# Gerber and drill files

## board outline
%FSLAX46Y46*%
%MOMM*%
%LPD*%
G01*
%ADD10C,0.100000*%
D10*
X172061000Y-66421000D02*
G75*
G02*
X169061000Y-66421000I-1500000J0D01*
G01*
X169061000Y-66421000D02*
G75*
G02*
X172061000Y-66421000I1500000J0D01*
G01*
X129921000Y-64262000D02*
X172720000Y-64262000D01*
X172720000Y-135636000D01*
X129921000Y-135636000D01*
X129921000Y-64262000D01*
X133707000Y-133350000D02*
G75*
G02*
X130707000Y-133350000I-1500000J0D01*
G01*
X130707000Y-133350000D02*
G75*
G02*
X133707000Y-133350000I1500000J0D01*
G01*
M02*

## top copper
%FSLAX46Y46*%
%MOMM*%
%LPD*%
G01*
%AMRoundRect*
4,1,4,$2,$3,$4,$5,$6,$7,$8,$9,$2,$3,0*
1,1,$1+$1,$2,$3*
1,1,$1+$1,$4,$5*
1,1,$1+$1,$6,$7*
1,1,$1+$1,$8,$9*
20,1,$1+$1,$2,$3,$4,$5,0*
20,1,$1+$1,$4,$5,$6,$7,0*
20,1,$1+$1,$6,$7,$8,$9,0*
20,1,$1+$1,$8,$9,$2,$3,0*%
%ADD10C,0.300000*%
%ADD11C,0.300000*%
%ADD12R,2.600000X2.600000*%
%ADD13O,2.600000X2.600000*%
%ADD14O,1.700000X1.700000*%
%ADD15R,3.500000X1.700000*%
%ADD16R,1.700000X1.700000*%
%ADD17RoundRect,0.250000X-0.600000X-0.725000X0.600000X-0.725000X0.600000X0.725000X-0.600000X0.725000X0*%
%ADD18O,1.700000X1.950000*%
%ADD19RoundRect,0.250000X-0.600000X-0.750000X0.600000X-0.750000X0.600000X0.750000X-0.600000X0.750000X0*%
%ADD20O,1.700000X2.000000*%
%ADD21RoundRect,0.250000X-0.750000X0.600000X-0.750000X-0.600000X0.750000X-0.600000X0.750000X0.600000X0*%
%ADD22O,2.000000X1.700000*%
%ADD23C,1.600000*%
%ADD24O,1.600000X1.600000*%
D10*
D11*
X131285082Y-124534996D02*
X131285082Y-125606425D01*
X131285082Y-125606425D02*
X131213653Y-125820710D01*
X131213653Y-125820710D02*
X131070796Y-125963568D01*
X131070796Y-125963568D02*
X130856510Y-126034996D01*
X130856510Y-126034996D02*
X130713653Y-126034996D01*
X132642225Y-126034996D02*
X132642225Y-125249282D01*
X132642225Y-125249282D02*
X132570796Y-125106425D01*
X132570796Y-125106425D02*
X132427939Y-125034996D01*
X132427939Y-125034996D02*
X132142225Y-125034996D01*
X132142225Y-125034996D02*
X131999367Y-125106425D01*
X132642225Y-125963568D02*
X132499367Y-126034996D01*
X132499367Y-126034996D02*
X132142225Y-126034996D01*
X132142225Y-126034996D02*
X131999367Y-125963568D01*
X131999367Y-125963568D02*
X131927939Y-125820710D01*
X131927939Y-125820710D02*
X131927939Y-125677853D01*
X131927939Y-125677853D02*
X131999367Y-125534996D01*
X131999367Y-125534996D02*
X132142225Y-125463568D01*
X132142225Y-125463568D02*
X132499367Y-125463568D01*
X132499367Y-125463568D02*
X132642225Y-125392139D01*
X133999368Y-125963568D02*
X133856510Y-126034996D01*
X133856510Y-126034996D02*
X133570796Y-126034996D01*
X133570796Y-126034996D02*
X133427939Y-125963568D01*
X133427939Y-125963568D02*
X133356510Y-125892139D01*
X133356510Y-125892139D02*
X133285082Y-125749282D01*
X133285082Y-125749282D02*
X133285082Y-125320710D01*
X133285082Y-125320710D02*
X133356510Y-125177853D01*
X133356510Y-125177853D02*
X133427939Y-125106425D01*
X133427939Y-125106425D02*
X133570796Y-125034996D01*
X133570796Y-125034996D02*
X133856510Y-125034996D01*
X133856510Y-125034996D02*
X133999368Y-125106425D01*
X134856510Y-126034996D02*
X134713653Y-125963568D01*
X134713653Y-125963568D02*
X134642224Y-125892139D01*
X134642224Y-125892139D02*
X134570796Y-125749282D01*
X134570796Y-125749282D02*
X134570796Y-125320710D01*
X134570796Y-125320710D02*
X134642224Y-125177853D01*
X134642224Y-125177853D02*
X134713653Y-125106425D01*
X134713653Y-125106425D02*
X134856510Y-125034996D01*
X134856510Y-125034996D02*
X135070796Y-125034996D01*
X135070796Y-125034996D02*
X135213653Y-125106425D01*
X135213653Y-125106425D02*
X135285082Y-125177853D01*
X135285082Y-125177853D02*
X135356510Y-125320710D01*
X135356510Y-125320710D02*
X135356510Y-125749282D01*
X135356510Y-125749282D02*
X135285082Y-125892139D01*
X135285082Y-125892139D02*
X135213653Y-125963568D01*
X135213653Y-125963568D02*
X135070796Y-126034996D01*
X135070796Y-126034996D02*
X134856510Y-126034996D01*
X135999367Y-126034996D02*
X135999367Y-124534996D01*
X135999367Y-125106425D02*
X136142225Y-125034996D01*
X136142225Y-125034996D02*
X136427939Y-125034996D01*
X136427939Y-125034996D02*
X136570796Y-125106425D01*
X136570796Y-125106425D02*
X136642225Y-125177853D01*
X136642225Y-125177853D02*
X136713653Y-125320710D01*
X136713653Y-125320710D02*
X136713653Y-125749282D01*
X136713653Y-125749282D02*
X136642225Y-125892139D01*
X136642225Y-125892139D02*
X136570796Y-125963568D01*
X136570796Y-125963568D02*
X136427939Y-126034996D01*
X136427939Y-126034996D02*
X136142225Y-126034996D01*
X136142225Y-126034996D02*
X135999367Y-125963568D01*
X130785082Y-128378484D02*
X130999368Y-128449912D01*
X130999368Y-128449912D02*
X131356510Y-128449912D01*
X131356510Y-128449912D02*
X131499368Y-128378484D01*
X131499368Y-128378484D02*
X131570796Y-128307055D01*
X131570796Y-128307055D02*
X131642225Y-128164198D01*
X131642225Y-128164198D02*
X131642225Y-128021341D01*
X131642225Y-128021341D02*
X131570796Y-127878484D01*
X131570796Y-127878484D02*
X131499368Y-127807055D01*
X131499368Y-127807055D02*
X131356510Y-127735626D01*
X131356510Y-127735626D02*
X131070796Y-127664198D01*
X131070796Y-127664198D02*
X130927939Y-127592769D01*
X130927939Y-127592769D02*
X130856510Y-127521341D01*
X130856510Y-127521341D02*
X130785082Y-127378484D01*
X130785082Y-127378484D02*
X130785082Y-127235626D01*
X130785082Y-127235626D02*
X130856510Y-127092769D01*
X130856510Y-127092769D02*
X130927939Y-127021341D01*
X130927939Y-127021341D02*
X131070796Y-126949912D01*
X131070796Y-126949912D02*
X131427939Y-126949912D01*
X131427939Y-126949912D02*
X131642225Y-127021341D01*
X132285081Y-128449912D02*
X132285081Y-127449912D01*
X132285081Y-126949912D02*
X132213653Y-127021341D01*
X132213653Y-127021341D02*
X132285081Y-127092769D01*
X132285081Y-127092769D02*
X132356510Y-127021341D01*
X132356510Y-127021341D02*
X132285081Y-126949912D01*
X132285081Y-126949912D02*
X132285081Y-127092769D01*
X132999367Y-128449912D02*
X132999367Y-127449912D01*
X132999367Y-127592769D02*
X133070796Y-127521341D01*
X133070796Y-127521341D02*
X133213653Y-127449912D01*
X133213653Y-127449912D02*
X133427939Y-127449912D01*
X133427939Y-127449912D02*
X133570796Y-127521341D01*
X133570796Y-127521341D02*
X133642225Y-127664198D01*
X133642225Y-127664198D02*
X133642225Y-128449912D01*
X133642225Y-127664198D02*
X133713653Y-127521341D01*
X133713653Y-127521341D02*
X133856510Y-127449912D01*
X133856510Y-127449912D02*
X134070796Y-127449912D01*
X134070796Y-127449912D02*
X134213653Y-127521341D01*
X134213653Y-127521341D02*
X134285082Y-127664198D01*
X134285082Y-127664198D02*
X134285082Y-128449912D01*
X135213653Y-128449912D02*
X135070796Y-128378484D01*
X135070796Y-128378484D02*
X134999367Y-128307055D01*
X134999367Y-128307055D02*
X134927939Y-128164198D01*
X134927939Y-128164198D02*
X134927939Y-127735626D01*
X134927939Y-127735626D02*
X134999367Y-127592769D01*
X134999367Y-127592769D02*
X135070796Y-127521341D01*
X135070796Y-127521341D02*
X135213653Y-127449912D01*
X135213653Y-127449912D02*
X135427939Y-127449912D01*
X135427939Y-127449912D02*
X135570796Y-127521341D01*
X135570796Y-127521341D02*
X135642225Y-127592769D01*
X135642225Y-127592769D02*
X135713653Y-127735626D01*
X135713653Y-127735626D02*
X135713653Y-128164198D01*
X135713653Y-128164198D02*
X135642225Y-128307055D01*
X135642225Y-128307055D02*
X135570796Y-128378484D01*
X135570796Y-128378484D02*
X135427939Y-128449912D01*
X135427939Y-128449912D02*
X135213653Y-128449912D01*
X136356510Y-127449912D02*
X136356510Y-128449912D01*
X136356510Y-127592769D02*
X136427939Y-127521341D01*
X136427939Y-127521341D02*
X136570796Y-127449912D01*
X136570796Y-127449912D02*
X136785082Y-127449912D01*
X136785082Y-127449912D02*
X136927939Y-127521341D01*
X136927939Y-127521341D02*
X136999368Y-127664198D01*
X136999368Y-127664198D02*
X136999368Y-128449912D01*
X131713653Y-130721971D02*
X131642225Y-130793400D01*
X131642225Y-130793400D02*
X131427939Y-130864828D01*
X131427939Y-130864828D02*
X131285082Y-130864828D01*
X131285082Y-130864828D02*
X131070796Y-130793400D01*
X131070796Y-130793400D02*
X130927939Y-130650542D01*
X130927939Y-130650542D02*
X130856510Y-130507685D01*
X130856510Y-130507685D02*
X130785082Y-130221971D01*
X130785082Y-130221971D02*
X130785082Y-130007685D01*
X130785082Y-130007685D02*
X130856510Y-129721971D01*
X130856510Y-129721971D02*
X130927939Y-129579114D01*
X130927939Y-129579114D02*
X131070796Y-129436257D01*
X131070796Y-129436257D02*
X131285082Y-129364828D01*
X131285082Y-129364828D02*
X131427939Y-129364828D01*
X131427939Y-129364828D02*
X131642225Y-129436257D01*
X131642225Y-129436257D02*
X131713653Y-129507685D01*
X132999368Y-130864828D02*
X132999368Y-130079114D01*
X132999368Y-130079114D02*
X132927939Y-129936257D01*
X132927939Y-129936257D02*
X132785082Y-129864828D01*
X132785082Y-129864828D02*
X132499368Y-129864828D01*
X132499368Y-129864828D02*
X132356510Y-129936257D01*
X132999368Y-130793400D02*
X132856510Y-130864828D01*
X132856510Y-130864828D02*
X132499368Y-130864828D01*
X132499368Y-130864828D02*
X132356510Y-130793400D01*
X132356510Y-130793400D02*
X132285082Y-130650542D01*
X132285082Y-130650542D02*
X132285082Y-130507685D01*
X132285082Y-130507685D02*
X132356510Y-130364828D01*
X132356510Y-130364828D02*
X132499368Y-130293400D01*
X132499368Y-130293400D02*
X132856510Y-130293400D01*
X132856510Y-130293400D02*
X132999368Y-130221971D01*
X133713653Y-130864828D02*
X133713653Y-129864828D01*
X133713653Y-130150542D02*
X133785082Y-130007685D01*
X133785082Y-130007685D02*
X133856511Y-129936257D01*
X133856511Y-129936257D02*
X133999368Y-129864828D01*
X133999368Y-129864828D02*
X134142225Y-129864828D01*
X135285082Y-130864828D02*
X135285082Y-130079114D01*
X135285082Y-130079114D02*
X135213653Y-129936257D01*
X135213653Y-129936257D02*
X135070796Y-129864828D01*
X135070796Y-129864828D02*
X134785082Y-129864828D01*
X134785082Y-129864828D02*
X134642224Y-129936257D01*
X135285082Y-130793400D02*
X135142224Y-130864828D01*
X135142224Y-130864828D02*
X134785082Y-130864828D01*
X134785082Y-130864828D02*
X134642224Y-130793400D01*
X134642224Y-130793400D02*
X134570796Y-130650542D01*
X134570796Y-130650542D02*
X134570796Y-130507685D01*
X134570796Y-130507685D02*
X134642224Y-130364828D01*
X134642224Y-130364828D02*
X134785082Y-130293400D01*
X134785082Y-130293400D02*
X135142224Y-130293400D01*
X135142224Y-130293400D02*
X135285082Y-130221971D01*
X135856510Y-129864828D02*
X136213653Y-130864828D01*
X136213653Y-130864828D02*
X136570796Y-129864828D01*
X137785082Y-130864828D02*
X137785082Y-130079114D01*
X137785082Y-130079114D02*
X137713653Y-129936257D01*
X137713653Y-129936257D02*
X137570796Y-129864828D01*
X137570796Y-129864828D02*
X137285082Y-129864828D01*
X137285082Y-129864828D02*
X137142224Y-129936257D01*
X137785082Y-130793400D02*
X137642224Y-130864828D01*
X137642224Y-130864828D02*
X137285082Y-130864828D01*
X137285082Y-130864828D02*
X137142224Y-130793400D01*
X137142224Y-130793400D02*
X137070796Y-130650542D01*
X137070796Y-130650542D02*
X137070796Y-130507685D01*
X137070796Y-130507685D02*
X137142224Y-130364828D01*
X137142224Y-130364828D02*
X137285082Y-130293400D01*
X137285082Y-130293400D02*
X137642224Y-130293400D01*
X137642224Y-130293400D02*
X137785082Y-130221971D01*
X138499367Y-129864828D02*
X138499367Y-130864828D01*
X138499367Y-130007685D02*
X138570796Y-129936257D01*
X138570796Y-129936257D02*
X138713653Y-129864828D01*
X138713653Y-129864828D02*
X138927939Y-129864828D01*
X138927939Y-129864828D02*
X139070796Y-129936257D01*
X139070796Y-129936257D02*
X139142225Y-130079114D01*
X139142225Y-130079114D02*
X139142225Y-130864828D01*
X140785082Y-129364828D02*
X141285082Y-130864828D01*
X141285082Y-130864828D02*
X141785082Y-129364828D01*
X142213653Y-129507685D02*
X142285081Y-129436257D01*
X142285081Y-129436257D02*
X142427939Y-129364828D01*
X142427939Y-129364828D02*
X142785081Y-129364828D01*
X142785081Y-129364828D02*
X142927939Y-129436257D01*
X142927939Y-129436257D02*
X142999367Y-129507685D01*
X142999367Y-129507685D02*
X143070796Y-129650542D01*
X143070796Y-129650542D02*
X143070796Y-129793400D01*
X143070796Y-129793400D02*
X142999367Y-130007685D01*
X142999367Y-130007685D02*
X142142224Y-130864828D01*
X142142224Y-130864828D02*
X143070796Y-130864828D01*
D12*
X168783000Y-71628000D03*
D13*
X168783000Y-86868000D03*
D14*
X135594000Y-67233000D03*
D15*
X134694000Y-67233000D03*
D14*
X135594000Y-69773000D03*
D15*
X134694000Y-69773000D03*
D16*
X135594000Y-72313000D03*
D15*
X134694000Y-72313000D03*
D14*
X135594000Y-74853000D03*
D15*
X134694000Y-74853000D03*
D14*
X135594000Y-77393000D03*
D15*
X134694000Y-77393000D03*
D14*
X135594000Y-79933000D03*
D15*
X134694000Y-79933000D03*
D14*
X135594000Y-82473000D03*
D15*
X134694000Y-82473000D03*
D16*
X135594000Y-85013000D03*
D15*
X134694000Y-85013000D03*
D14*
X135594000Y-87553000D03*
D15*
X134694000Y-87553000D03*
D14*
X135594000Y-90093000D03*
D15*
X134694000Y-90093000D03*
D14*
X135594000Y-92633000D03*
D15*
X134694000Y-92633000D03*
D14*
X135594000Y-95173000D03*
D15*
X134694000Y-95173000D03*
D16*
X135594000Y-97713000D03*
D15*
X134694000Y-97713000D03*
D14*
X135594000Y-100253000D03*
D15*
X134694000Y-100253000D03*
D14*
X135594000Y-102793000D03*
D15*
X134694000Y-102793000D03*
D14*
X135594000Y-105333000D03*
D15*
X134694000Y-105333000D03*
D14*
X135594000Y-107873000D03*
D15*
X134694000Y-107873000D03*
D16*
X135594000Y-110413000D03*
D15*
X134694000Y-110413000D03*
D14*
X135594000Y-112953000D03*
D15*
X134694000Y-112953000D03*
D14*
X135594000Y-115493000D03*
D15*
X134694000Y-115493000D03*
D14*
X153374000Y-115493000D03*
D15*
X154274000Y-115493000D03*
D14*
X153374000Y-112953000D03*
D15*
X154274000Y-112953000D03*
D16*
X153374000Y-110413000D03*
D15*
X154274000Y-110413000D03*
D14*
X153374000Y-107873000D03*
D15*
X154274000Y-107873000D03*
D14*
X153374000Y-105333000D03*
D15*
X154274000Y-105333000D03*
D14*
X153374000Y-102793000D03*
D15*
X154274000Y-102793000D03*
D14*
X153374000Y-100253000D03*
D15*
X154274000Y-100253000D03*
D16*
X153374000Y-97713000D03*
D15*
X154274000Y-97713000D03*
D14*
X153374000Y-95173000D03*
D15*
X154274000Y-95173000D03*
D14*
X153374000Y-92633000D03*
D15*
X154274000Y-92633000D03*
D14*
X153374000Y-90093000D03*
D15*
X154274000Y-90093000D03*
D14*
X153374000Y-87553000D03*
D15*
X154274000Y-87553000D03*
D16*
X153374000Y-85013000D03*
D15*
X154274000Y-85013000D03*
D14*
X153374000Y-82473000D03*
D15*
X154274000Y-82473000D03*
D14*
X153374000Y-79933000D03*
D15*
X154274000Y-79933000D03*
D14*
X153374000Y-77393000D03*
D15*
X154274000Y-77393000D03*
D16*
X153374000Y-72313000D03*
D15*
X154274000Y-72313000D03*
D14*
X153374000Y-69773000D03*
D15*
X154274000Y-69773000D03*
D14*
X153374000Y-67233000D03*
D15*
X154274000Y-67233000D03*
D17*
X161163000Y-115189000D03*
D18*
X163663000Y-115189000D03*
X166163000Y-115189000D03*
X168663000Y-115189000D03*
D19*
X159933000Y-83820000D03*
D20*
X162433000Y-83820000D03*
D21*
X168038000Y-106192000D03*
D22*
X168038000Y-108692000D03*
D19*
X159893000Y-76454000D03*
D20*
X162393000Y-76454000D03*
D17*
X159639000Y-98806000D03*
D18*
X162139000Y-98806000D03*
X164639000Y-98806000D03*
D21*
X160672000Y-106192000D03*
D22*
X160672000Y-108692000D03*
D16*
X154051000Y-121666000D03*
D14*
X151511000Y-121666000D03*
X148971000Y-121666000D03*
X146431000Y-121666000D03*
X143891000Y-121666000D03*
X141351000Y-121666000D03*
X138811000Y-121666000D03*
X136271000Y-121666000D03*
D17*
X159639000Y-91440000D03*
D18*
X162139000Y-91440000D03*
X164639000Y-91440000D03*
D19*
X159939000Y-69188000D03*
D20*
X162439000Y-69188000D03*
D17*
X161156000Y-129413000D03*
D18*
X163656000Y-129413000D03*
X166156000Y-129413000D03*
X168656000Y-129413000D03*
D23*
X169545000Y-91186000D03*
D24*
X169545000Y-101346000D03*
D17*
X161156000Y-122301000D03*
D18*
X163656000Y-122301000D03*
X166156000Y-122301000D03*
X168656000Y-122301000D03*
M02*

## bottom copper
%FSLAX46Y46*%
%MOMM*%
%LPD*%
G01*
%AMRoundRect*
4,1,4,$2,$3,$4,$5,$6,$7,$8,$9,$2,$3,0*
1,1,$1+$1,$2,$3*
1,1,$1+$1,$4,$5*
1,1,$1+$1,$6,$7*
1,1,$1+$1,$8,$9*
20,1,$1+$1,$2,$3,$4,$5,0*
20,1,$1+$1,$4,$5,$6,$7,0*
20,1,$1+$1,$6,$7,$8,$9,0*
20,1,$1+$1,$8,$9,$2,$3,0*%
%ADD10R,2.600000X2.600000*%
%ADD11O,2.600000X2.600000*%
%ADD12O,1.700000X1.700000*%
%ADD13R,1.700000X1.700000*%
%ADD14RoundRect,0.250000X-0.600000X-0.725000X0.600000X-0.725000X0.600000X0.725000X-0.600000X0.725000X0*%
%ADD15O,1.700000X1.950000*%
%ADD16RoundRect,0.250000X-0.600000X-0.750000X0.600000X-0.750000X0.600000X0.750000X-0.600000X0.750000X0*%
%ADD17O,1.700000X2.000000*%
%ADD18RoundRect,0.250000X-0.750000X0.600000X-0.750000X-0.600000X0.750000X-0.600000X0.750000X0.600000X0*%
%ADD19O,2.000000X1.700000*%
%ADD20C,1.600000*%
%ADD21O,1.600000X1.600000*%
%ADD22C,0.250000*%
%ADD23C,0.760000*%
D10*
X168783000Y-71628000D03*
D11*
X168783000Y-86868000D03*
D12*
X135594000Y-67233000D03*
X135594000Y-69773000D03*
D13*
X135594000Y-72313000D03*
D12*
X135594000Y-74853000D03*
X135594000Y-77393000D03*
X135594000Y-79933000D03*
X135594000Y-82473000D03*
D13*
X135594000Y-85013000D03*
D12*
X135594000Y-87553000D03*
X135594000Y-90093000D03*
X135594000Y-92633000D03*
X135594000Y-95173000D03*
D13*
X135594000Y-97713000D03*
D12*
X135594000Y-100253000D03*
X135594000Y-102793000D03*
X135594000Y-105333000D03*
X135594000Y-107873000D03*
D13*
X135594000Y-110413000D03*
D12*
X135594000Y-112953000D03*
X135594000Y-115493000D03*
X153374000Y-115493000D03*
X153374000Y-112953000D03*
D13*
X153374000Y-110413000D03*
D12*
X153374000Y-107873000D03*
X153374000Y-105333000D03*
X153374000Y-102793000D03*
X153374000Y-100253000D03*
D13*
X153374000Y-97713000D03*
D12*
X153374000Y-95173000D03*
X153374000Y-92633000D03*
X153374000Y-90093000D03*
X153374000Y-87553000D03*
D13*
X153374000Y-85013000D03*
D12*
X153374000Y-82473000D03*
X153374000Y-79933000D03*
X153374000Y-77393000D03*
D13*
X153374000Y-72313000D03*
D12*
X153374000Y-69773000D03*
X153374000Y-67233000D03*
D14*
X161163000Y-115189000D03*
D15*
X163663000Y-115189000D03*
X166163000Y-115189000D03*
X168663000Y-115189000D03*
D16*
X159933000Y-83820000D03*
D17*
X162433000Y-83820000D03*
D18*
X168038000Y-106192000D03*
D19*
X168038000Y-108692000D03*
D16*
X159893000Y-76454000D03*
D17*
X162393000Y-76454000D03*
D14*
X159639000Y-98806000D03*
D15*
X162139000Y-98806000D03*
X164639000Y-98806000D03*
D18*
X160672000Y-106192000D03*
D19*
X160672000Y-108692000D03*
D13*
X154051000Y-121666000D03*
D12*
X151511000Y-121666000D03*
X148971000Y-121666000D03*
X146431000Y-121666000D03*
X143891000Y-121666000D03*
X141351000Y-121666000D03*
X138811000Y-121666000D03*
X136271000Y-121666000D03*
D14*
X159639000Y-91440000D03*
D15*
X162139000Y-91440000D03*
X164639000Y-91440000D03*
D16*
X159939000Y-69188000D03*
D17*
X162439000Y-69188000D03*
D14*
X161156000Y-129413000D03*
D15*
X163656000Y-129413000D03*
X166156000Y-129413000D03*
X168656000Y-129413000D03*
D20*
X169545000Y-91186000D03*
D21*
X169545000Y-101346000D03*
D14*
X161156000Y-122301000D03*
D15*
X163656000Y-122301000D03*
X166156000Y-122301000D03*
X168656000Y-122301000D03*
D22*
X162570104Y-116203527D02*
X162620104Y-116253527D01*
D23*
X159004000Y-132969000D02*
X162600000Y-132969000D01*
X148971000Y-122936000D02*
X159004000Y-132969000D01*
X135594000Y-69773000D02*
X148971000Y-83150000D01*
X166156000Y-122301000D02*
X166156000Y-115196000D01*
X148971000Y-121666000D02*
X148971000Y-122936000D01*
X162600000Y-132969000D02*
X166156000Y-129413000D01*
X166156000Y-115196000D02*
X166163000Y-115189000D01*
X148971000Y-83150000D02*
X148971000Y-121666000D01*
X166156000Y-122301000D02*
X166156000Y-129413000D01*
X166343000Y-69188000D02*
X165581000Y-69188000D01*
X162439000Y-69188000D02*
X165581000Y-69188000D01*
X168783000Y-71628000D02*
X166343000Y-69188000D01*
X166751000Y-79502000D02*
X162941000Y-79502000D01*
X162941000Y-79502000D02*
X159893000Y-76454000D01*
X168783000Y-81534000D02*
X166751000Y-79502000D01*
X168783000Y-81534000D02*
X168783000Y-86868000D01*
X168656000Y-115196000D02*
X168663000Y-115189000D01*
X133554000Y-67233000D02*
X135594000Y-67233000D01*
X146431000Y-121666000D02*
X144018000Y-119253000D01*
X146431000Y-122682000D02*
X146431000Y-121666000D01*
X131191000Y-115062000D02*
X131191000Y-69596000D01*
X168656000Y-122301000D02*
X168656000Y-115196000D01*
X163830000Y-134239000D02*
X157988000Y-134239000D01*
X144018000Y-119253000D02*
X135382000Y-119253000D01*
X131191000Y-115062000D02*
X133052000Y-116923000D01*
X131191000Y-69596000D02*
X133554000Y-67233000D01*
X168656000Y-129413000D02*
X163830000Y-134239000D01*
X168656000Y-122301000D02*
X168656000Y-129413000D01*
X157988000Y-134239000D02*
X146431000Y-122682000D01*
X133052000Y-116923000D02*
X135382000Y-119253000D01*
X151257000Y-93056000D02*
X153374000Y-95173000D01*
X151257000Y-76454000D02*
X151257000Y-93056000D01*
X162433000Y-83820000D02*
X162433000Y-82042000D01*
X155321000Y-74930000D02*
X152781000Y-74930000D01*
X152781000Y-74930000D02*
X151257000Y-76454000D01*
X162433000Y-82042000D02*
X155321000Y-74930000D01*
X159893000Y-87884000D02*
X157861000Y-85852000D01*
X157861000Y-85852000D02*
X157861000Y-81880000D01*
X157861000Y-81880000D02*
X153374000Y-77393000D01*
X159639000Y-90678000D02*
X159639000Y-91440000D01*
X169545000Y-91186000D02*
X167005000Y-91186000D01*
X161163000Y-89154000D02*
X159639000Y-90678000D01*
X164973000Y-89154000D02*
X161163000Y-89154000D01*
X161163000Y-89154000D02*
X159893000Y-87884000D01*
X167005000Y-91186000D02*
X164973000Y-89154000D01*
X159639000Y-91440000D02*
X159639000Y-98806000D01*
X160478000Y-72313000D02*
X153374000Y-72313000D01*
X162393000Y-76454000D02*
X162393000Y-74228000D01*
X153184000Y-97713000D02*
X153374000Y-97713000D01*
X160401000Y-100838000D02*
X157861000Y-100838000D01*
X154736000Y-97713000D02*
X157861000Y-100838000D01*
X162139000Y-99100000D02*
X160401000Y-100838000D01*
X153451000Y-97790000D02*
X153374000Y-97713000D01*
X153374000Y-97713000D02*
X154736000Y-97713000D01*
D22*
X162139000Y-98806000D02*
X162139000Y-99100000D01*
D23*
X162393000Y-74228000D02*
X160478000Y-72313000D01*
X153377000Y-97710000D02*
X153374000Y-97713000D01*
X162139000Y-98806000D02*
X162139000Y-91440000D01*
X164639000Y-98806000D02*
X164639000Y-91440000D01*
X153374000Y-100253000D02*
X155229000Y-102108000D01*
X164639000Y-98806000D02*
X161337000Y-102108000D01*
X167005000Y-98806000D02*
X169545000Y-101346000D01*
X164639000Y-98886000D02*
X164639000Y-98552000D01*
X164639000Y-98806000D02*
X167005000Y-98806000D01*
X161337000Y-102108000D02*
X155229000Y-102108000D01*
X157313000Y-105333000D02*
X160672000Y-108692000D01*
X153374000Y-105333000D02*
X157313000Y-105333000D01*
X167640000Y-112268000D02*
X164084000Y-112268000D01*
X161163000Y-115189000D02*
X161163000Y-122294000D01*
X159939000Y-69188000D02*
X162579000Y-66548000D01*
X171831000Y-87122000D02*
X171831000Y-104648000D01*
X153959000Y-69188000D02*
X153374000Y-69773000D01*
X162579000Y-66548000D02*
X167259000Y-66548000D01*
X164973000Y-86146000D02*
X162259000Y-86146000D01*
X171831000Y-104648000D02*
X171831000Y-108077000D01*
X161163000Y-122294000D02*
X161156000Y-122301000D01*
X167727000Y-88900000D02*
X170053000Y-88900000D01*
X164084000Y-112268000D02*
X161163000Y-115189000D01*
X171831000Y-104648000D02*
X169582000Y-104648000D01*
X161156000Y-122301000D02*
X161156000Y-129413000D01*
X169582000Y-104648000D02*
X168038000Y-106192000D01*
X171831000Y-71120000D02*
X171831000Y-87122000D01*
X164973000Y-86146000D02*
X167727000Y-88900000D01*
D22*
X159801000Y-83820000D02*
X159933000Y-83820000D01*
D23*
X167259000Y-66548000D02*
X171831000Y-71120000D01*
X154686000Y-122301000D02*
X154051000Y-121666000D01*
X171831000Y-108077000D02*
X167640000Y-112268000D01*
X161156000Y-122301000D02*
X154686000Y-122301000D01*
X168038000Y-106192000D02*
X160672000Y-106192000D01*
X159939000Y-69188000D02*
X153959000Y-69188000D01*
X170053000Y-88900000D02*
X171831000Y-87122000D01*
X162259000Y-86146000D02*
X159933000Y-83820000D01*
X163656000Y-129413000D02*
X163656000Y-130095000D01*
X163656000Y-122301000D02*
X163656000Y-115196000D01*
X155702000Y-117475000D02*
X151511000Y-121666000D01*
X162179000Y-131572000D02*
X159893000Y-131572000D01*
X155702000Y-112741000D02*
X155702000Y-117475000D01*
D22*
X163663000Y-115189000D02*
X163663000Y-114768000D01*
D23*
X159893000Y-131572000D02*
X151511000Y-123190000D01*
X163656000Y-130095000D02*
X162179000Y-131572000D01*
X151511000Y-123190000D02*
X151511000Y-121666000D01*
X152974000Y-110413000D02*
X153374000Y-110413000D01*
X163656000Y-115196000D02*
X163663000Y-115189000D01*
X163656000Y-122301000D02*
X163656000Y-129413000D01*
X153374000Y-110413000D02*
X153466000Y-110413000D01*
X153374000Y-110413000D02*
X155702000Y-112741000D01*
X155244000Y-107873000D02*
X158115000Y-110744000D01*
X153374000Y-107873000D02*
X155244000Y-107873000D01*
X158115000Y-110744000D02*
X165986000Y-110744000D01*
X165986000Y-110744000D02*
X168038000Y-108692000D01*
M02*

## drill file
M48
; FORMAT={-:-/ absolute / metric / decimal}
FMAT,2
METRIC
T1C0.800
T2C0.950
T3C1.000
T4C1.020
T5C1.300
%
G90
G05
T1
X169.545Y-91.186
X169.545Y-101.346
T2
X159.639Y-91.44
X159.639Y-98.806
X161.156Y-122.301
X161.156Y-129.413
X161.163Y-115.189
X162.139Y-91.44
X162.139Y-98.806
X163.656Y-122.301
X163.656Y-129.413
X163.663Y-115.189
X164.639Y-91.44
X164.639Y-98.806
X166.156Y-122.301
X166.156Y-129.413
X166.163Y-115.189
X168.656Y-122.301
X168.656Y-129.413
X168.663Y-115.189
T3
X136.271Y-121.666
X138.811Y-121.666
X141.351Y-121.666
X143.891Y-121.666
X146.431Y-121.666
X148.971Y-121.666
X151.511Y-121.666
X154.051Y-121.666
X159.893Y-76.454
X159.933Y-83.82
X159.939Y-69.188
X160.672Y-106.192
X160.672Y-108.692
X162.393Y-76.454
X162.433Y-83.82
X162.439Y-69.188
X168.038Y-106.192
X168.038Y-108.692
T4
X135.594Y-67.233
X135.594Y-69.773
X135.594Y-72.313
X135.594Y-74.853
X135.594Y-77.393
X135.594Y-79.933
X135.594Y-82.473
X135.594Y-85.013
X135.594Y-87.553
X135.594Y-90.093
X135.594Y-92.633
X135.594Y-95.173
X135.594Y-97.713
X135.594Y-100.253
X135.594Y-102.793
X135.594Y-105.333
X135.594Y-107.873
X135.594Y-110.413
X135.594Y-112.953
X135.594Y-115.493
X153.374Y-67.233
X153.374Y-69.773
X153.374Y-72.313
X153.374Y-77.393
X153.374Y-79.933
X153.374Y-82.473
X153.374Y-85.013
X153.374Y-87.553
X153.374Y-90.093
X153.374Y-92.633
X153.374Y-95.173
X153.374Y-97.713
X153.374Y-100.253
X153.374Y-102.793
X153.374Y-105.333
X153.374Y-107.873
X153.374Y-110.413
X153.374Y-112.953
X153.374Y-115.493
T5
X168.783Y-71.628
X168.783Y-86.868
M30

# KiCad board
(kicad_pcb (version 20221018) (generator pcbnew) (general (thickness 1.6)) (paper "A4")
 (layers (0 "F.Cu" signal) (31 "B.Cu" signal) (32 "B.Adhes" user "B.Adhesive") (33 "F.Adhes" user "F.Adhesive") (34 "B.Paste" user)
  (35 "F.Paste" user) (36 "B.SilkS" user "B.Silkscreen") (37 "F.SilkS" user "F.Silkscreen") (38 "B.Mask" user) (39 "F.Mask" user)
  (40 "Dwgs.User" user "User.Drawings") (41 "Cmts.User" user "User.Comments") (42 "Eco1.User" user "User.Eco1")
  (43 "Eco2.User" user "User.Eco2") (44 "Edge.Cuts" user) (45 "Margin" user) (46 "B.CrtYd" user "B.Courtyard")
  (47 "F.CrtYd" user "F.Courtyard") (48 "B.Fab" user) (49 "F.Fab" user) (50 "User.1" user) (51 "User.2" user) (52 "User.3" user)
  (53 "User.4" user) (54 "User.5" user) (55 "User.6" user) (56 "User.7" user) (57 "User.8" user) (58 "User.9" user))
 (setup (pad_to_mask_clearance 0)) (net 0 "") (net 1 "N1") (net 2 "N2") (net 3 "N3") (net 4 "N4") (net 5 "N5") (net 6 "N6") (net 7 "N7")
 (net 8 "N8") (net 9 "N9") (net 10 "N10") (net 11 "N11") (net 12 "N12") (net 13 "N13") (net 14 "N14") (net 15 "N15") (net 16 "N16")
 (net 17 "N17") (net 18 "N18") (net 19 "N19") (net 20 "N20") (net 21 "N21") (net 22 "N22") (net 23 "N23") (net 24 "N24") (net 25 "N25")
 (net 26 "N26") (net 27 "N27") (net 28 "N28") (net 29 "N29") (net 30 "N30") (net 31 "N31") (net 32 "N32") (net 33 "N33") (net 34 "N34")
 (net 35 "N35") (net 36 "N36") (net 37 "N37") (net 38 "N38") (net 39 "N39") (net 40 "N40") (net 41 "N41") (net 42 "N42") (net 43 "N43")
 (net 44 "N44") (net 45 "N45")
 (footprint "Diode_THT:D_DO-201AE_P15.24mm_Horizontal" (layer "F.Cu") (at 168.783 71.628 -90)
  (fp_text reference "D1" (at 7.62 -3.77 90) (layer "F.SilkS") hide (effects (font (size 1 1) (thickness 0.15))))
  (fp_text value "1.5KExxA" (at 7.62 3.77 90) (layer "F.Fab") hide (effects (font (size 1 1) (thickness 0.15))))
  (pad "1" thru_hole rect (at 0 0 270) (size 2.6 2.6) (drill 1.3) (layers "*.Cu" "*.Mask") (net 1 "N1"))
  (pad "2" thru_hole oval (at 15.24 0 270) (size 2.6 2.6) (drill 1.3) (layers "*.Cu" "*.Mask") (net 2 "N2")))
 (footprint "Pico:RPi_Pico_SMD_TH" (layer "F.Cu") (at 144.484 91.363)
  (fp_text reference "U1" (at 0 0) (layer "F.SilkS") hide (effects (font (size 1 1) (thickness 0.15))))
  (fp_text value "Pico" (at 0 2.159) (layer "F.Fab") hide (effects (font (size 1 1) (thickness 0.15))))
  (pad "1" thru_hole oval (at -8.89 -24.13) (size 1.7 1.7) (drill 1.02) (layers "*.Cu" "*.Mask") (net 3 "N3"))
  (pad "1" smd rect (at -8.89 -24.13) (size 3.5 1.7) (drill (offset -0.9 0)) (layers "F.Cu" "F.Mask") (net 3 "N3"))
  (pad "2" thru_hole oval (at -8.89 -21.59) (size 1.7 1.7) (drill 1.02) (layers "*.Cu" "*.Mask") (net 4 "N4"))
  (pad "2" smd rect (at -8.89 -21.59) (size 3.5 1.7) (drill (offset -0.9 0)) (layers "F.Cu" "F.Mask") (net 4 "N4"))
  (pad "3" thru_hole rect (at -8.89 -19.05) (size 1.7 1.7) (drill 1.02) (layers "*.Cu" "*.Mask") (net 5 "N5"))
  (pad "3" smd rect (at -8.89 -19.05) (size 3.5 1.7) (drill (offset -0.9 0)) (layers "F.Cu" "F.Mask") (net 5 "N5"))
  (pad "4" thru_hole oval (at -8.89 -16.51) (size 1.7 1.7) (drill 1.02) (layers "*.Cu" "*.Mask") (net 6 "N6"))
  (pad "4" smd rect (at -8.89 -16.51) (size 3.5 1.7) (drill (offset -0.9 0)) (layers "F.Cu" "F.Mask") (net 6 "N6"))
  (pad "5" thru_hole oval (at -8.89 -13.97) (size 1.7 1.7) (drill 1.02) (layers "*.Cu" "*.Mask") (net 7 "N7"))
  (pad "5" smd rect (at -8.89 -13.97) (size 3.5 1.7) (drill (offset -0.9 0)) (layers "F.Cu" "F.Mask") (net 7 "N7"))
  (pad "6" thru_hole oval (at -8.89 -11.43) (size 1.7 1.7) (drill 1.02) (layers "*.Cu" "*.Mask") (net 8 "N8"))
  (pad "6" smd rect (at -8.89 -11.43) (size 3.5 1.7) (drill (offset -0.9 0)) (layers "F.Cu" "F.Mask") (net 8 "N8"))
  (pad "7" thru_hole oval (at -8.89 -8.89) (size 1.7 1.7) (drill 1.02) (layers "*.Cu" "*.Mask") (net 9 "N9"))
  (pad "7" smd rect (at -8.89 -8.89) (size 3.5 1.7) (drill (offset -0.9 0)) (layers "F.Cu" "F.Mask") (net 9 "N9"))
  (pad "8" thru_hole rect (at -8.89 -6.35) (size 1.7 1.7) (drill 1.02) (layers "*.Cu" "*.Mask") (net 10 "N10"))
  (pad "8" smd rect (at -8.89 -6.35) (size 3.5 1.7) (drill (offset -0.9 0)) (layers "F.Cu" "F.Mask") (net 10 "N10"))
  (pad "9" thru_hole oval (at -8.89 -3.81) (size 1.7 1.7) (drill 1.02) (layers "*.Cu" "*.Mask") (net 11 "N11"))
  (pad "9" smd rect (at -8.89 -3.81) (size 3.5 1.7) (drill (offset -0.9 0)) (layers "F.Cu" "F.Mask") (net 11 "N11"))
  (pad "10" thru_hole oval (at -8.89 -1.27) (size 1.7 1.7) (drill 1.02) (layers "*.Cu" "*.Mask") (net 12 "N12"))
  (pad "10" smd rect (at -8.89 -1.27) (size 3.5 1.7) (drill (offset -0.9 0)) (layers "F.Cu" "F.Mask") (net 12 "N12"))
  (pad "11" thru_hole oval (at -8.89 1.27) (size 1.7 1.7) (drill 1.02) (layers "*.Cu" "*.Mask") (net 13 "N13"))
  (pad "11" smd rect (at -8.89 1.27) (size 3.5 1.7) (drill (offset -0.9 0)) (layers "F.Cu" "F.Mask") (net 13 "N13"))
  (pad "12" thru_hole oval (at -8.89 3.81) (size 1.7 1.7) (drill 1.02) (layers "*.Cu" "*.Mask") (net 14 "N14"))
  (pad "12" smd rect (at -8.89 3.81) (size 3.5 1.7) (drill (offset -0.9 0)) (layers "F.Cu" "F.Mask") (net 14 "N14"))
  (pad "13" thru_hole rect (at -8.89 6.35) (size 1.7 1.7) (drill 1.02) (layers "*.Cu" "*.Mask") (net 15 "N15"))
  (pad "13" smd rect (at -8.89 6.35) (size 3.5 1.7) (drill (offset -0.9 0)) (layers "F.Cu" "F.Mask") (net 15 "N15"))
  (pad "14" thru_hole oval (at -8.89 8.89) (size 1.7 1.7) (drill 1.02) (layers "*.Cu" "*.Mask") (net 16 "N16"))
  (pad "14" smd rect (at -8.89 8.89) (size 3.5 1.7) (drill (offset -0.9 0)) (layers "F.Cu" "F.Mask") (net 16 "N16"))
  (pad "15" thru_hole oval (at -8.89 11.43) (size 1.7 1.7) (drill 1.02) (layers "*.Cu" "*.Mask") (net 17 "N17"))
  (pad "15" smd rect (at -8.89 11.43) (size 3.5 1.7) (drill (offset -0.9 0)) (layers "F.Cu" "F.Mask") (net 17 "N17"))
  (pad "16" thru_hole oval (at -8.89 13.97) (size 1.7 1.7) (drill 1.02) (layers "*.Cu" "*.Mask") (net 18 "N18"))
  (pad "16" smd rect (at -8.89 13.97) (size 3.5 1.7) (drill (offset -0.9 0)) (layers "F.Cu" "F.Mask") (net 18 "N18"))
  (pad "17" thru_hole oval (at -8.89 16.51) (size 1.7 1.7) (drill 1.02) (layers "*.Cu" "*.Mask") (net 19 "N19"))
  (pad "17" smd rect (at -8.89 16.51) (size 3.5 1.7) (drill (offset -0.9 0)) (layers "F.Cu" "F.Mask") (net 19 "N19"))
  (pad "18" thru_hole rect (at -8.89 19.05) (size 1.7 1.7) (drill 1.02) (layers "*.Cu" "*.Mask") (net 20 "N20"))
  (pad "18" smd rect (at -8.89 19.05) (size 3.5 1.7) (drill (offset -0.9 0)) (layers "F.Cu" "F.Mask") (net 20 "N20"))
  (pad "19" thru_hole oval (at -8.89 21.59) (size 1.7 1.7) (drill 1.02) (layers "*.Cu" "*.Mask") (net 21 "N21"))
  (pad "19" smd rect (at -8.89 21.59) (size 3.5 1.7) (drill (offset -0.9 0)) (layers "F.Cu" "F.Mask") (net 21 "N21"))
  (pad "20" thru_hole oval (at -8.89 24.13) (size 1.7 1.7) (drill 1.02) (layers "*.Cu" "*.Mask") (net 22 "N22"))
  (pad "20" smd rect (at -8.89 24.13) (size 3.5 1.7) (drill (offset -0.9 0)) (layers "F.Cu" "F.Mask") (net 22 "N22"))
  (pad "21" thru_hole oval (at 8.89 24.13) (size 1.7 1.7) (drill 1.02) (layers "*.Cu" "*.Mask") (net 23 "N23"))
  (pad "21" smd rect (at 8.89 24.13) (size 3.5 1.7) (drill (offset 0.9 0)) (layers "F.Cu" "F.Mask") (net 23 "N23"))
  (pad "22" thru_hole oval (at 8.89 21.59) (size 1.7 1.7) (drill 1.02) (layers "*.Cu" "*.Mask") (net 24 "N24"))
  (pad "22" smd rect (at 8.89 21.59) (size 3.5 1.7) (drill (offset 0.9 0)) (layers "F.Cu" "F.Mask") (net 24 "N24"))
  (pad "23" thru_hole rect (at 8.89 19.05) (size 1.7 1.7) (drill 1.02) (layers "*.Cu" "*.Mask") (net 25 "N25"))
  (pad "23" smd rect (at 8.89 19.05) (size 3.5 1.7) (drill (offset 0.9 0)) (layers "F.Cu" "F.Mask") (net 25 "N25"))
  (pad "24" thru_hole oval (at 8.89 16.51) (size 1.7 1.7) (drill 1.02) (layers "*.Cu" "*.Mask") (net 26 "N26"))
  (pad "24" smd rect (at 8.89 16.51) (size 3.5 1.7) (drill (offset 0.9 0)) (layers "F.Cu" "F.Mask") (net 26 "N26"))
  (pad "25" thru_hole oval (at 8.89 13.97) (size 1.7 1.7) (drill 1.02) (layers "*.Cu" "*.Mask") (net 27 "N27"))
  (pad "25" smd rect (at 8.89 13.97) (size 3.5 1.7) (drill (offset 0.9 0)) (layers "F.Cu" "F.Mask") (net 27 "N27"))
  (pad "26" thru_hole oval (at 8.89 11.43) (size 1.7 1.7) (drill 1.02) (layers "*.Cu" "*.Mask") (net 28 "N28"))
  (pad "26" smd rect (at 8.89 11.43) (size 3.5 1.7) (drill (offset 0.9 0)) (layers "F.Cu" "F.Mask") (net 28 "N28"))
  (pad "27" thru_hole oval (at 8.89 8.89) (size 1.7 1.7) (drill 1.02) (layers "*.Cu" "*.Mask") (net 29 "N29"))
  (pad "27" smd rect (at 8.89 8.89) (size 3.5 1.7) (drill (offset 0.9 0)) (layers "F.Cu" "F.Mask") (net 29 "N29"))
  (pad "28" thru_hole rect (at 8.89 6.35) (size 1.7 1.7) (drill 1.02) (layers "*.Cu" "*.Mask") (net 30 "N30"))
  (pad "28" smd rect (at 8.89 6.35) (size 3.5 1.7) (drill (offset 0.9 0)) (layers "F.Cu" "F.Mask") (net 30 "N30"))
  (pad "29" thru_hole oval (at 8.89 3.81) (size 1.7 1.7) (drill 1.02) (layers "*.Cu" "*.Mask") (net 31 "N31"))
  (pad "29" smd rect (at 8.89 3.81) (size 3.5 1.7) (drill (offset 0.9 0)) (layers "F.Cu" "F.Mask") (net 31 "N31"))
  (pad "30" thru_hole oval (at 8.89 1.27) (size 1.7 1.7) (drill 1.02) (layers "*.Cu" "*.Mask") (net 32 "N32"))
  (pad "30" smd rect (at 8.89 1.27) (size 3.5 1.7) (drill (offset 0.9 0)) (layers "F.Cu" "F.Mask") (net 32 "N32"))
  (pad "31" thru_hole oval (at 8.89 -1.27) (size 1.7 1.7) (drill 1.02) (layers "*.Cu" "*.Mask") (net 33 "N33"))
  (pad "31" smd rect (at 8.89 -1.27) (size 3.5 1.7) (drill (offset 0.9 0)) (layers "F.Cu" "F.Mask") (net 33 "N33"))
  (pad "32" thru_hole oval (at 8.89 -3.81) (size 1.7 1.7) (drill 1.02) (layers "*.Cu" "*.Mask") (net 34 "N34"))
  (pad "32" smd rect (at 8.89 -3.81) (size 3.5 1.7) (drill (offset 0.9 0)) (layers "F.Cu" "F.Mask") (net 34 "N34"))
  (pad "33" thru_hole rect (at 8.89 -6.35) (size 1.7 1.7) (drill 1.02) (layers "*.Cu" "*.Mask") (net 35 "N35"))
  (pad "33" smd rect (at 8.89 -6.35) (size 3.5 1.7) (drill (offset 0.9 0)) (layers "F.Cu" "F.Mask") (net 35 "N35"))
  (pad "34" thru_hole oval (at 8.89 -8.89) (size 1.7 1.7) (drill 1.02) (layers "*.Cu" "*.Mask") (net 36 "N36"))
  (pad "34" smd rect (at 8.89 -8.89) (size 3.5 1.7) (drill (offset 0.9 0)) (layers "F.Cu" "F.Mask") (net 36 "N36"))
  (pad "35" thru_hole oval (at 8.89 -11.43) (size 1.7 1.7) (drill 1.02) (layers "*.Cu" "*.Mask") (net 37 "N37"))
  (pad "35" smd rect (at 8.89 -11.43) (size 3.5 1.7) (drill (offset 0.9 0)) (layers "F.Cu" "F.Mask") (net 37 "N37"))
  (pad "36" thru_hole oval (at 8.89 -13.97) (size 1.7 1.7) (drill 1.02) (layers "*.Cu" "*.Mask") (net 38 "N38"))
  (pad "36" smd rect (at 8.89 -13.97) (size 3.5 1.7) (drill (offset 0.9 0)) (layers "F.Cu" "F.Mask") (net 38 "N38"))
  (pad "38" thru_hole rect (at 8.89 -19.05) (size 1.7 1.7) (drill 1.02) (layers "*.Cu" "*.Mask") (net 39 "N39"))
  (pad "38" smd rect (at 8.89 -19.05) (size 3.5 1.7) (drill (offset 0.9 0)) (layers "F.Cu" "F.Mask") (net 39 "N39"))
  (pad "39" thru_hole oval (at 8.89 -21.59) (size 1.7 1.7) (drill 1.02) (layers "*.Cu" "*.Mask") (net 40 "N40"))
  (pad "39" smd rect (at 8.89 -21.59) (size 3.5 1.7) (drill (offset 0.9 0)) (layers "F.Cu" "F.Mask") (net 40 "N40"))
  (pad "40" thru_hole oval (at 8.89 -24.13) (size 1.7 1.7) (drill 1.02) (layers "*.Cu" "*.Mask") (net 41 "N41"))
  (pad "40" smd rect (at 8.89 -24.13) (size 3.5 1.7) (drill (offset 0.9 0)) (layers "F.Cu" "F.Mask") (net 41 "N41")))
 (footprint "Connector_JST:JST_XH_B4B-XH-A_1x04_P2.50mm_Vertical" (layer "F.Cu") (at 161.163 115.189)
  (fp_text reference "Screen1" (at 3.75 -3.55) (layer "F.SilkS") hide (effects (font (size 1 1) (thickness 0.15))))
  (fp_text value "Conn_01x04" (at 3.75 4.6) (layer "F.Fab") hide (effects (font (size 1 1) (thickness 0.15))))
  (pad "1" thru_hole roundrect (at 0 0) (size 1.7 1.95) (drill 0.95) (layers "*.Cu" "*.Mask") (roundrect_rratio 0.1470588235) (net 40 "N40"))
  (pad "2" thru_hole oval (at 2.5 0) (size 1.7 1.95) (drill 0.95) (layers "*.Cu" "*.Mask") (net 25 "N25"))
  (pad "3" thru_hole oval (at 5 0) (size 1.7 1.95) (drill 0.95) (layers "*.Cu" "*.Mask") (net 4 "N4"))
  (pad "4" thru_hole oval (at 7.5 0) (size 1.7 1.95) (drill 0.95) (layers "*.Cu" "*.Mask") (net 3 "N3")))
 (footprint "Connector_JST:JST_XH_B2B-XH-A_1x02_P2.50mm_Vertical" (layer "F.Cu") (at 159.933 83.82)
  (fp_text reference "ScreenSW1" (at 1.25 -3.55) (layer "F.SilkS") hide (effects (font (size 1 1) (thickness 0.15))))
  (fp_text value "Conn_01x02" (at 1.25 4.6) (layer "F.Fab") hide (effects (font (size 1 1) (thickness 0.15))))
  (pad "1" thru_hole roundrect (at 0 0) (size 1.7 2) (drill 1) (layers "*.Cu" "*.Mask") (roundrect_rratio 0.1470588235) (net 40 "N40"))
  (pad "2" thru_hole oval (at 2.5 0) (size 1.7 2) (drill 1) (layers "*.Cu" "*.Mask") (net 31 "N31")))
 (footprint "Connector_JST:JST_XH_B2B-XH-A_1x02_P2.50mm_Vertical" (layer "F.Cu") (at 168.038 106.192 -90)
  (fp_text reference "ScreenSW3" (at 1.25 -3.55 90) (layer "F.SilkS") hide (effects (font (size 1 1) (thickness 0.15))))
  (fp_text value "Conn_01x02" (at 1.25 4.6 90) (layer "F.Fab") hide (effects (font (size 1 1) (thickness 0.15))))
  (pad "1" thru_hole roundrect (at 0 0 270) (size 1.7 2) (drill 1) (layers "*.Cu" "*.Mask") (roundrect_rratio 0.1470588235) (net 40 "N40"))
  (pad "2" thru_hole oval (at 2.5 0 270) (size 1.7 2) (drill 1) (layers "*.Cu" "*.Mask") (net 26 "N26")))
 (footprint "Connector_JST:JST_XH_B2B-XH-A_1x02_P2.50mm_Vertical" (layer "F.Cu") (at 159.893 76.454)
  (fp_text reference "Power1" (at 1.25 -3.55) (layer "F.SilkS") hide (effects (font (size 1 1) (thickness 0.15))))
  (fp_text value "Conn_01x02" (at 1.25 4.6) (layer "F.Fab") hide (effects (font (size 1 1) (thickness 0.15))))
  (pad "1" thru_hole roundrect (at 0 0) (size 1.7 2) (drill 1) (layers "*.Cu" "*.Mask") (roundrect_rratio 0.1470588235) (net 2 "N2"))
  (pad "2" thru_hole oval (at 2.5 0) (size 1.7 2) (drill 1) (layers "*.Cu" "*.Mask") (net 25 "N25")))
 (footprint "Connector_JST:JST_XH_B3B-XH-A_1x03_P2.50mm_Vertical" (layer "F.Cu") (at 159.639 98.806)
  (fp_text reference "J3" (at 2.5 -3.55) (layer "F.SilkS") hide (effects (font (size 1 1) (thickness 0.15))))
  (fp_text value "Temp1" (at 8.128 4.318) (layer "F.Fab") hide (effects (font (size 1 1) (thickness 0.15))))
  (pad "1" thru_hole roundrect (at 0 0) (size 1.7 1.95) (drill 0.95) (layers "*.Cu" "*.Mask") (roundrect_rratio 0.1470588235) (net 38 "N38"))
  (pad "2" thru_hole oval (at 2.5 0) (size 1.7 1.95) (drill 0.95) (layers "*.Cu" "*.Mask") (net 30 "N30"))
  (pad "3" thru_hole oval (at 5 0) (size 1.7 1.95) (drill 0.95) (layers "*.Cu" "*.Mask") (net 29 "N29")))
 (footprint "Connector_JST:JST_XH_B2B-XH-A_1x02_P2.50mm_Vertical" (layer "F.Cu") (at 160.672 106.192 -90)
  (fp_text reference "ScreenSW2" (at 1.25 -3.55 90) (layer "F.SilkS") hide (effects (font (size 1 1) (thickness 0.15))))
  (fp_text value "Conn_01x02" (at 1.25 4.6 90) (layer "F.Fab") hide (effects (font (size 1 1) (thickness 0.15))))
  (pad "1" thru_hole roundrect (at 0 0 270) (size 1.7 2) (drill 1) (layers "*.Cu" "*.Mask") (roundrect_rratio 0.1470588235) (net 40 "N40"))
  (pad "2" thru_hole oval (at 2.5 0 270) (size 1.7 2) (drill 1) (layers "*.Cu" "*.Mask") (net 27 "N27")))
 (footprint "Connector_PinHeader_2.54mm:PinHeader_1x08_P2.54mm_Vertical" (layer "F.Cu") (at 154.051 121.666 -90)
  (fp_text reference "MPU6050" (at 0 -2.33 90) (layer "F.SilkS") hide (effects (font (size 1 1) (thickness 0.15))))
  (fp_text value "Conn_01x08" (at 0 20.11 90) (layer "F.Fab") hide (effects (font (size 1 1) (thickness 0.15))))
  (pad "1" thru_hole rect (at 0 0 270) (size 1.7 1.7) (drill 1) (layers "*.Cu" "*.Mask") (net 40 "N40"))
  (pad "2" thru_hole oval (at 0 2.54 270) (size 1.7 1.7) (drill 1) (layers "*.Cu" "*.Mask") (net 25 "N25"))
  (pad "3" thru_hole oval (at 0 5.08 270) (size 1.7 1.7) (drill 1) (layers "*.Cu" "*.Mask") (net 4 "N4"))
  (pad "4" thru_hole oval (at 0 7.62 270) (size 1.7 1.7) (drill 1) (layers "*.Cu" "*.Mask") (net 3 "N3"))
  (pad "5" thru_hole oval (at 0 10.16 270) (size 1.7 1.7) (drill 1) (layers "*.Cu" "*.Mask") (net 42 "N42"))
  (pad "6" thru_hole oval (at 0 12.7 270) (size 1.7 1.7) (drill 1) (layers "*.Cu" "*.Mask") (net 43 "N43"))
  (pad "7" thru_hole oval (at 0 15.24 270) (size 1.7 1.7) (drill 1) (layers "*.Cu" "*.Mask") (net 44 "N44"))
  (pad "8" thru_hole oval (at 0 17.78 270) (size 1.7 1.7) (drill 1) (layers "*.Cu" "*.Mask") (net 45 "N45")))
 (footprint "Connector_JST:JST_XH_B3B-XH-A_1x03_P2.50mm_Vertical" (layer "F.Cu") (at 159.639 91.44)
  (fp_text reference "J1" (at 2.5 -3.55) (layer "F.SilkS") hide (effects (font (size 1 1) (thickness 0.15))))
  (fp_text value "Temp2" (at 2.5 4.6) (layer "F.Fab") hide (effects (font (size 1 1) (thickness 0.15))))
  (pad "1" thru_hole roundrect (at 0 0) (size 1.7 1.95) (drill 0.95) (layers "*.Cu" "*.Mask") (roundrect_rratio 0.1470588235) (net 38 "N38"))
  (pad "2" thru_hole oval (at 2.5 0) (size 1.7 1.95) (drill 0.95) (layers "*.Cu" "*.Mask") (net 30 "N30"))
  (pad "3" thru_hole oval (at 5 0) (size 1.7 1.95) (drill 0.95) (layers "*.Cu" "*.Mask") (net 29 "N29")))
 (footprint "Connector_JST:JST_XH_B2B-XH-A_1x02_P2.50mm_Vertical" (layer "F.Cu") (at 159.939 69.188)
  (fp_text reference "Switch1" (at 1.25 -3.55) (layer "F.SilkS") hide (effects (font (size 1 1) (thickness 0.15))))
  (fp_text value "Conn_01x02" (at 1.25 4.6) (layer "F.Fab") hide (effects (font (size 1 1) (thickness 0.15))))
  (pad "1" thru_hole roundrect (at 0 0) (size 1.7 2) (drill 1) (layers "*.Cu" "*.Mask") (roundrect_rratio 0.1470588235) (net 40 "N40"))
  (pad "2" thru_hole oval (at 2.5 0) (size 1.7 2) (drill 1) (layers "*.Cu" "*.Mask") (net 1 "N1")))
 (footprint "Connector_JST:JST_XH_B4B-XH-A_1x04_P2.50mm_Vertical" (layer "F.Cu") (at 161.156 129.413)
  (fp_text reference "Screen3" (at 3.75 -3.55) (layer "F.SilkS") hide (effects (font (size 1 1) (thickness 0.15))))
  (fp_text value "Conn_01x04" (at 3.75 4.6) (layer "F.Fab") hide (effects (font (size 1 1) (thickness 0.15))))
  (pad "1" thru_hole roundrect (at 0 0) (size 1.7 1.95) (drill 0.95) (layers "*.Cu" "*.Mask") (roundrect_rratio 0.1470588235) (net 40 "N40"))
  (pad "2" thru_hole oval (at 2.5 0) (size 1.7 1.95) (drill 0.95) (layers "*.Cu" "*.Mask") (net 25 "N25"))
  (pad "3" thru_hole oval (at 5 0) (size 1.7 1.95) (drill 0.95) (layers "*.Cu" "*.Mask") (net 4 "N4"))
  (pad "4" thru_hole oval (at 7.5 0) (size 1.7 1.95) (drill 0.95) (layers "*.Cu" "*.Mask") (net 3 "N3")))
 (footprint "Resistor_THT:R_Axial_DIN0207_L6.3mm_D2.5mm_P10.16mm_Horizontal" (layer "F.Cu") (at 169.545 91.186 -90)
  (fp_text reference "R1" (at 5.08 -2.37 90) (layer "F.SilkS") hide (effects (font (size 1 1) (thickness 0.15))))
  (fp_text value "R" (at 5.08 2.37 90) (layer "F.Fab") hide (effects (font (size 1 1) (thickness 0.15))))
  (pad "1" thru_hole circle (at 0 0 270) (size 1.6 1.6) (drill 0.8) (layers "*.Cu" "*.Mask") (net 38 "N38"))
  (pad "2" thru_hole oval (at 10.16 0 270) (size 1.6 1.6) (drill 0.8) (layers "*.Cu" "*.Mask") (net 29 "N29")))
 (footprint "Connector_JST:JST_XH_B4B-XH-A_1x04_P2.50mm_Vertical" (layer "F.Cu") (at 161.156 122.301)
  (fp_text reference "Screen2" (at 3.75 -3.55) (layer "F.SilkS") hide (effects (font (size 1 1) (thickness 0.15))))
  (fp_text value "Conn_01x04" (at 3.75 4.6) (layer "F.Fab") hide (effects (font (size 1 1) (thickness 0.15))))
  (pad "1" thru_hole roundrect (at 0 0) (size 1.7 1.95) (drill 0.95) (layers "*.Cu" "*.Mask") (roundrect_rratio 0.1470588235) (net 40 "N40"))
  (pad "2" thru_hole oval (at 2.5 0) (size 1.7 1.95) (drill 0.95) (layers "*.Cu" "*.Mask") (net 25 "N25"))
  (pad "3" thru_hole oval (at 5 0) (size 1.7 1.95) (drill 0.95) (layers "*.Cu" "*.Mask") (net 4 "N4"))
  (pad "4" thru_hole oval (at 7.5 0) (size 1.7 1.95) (drill 0.95) (layers "*.Cu" "*.Mask") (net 3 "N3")))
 (gr_circle (center 170.561 66.421) (end 172.061 66.421) (stroke (width 0.1) (type solid)) (fill none) (layer "Edge.Cuts"))
 (gr_rect (start 129.921 64.262) (end 172.72 135.636) (stroke (width 0.1) (type default)) (fill none) (layer "Edge.Cuts"))
 (gr_circle (center 132.207 133.35) (end 133.707 133.35) (stroke (width 0.1) (type solid)) (fill none) (layer "Edge.Cuts"))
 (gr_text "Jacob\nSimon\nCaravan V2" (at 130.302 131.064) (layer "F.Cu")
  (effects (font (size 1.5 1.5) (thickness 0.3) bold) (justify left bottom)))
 (segment (start 162.570104 116.203527) (end 162.620104 116.253527) (width 0.25) (layer "B.Cu") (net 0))
 (segment (start 159.004 132.969) (end 162.6 132.969) (width 0.76) (layer "B.Cu") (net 4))
 (segment (start 148.971 122.936) (end 159.004 132.969) (width 0.76) (layer "B.Cu") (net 4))
 (segment (start 135.594 69.773) (end 148.971 83.15) (width 0.76) (layer "B.Cu") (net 4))
 (segment (start 166.156 122.301) (end 166.156 115.196) (width 0.76) (layer "B.Cu") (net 4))
 (segment (start 148.971 121.666) (end 148.971 122.936) (width 0.76) (layer "B.Cu") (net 4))
 (segment (start 162.6 132.969) (end 166.156 129.413) (width 0.76) (layer "B.Cu") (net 4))
 (segment (start 166.156 115.196) (end 166.163 115.189) (width 0.76) (layer "B.Cu") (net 4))
 (segment (start 148.971 83.15) (end 148.971 121.666) (width 0.76) (layer "B.Cu") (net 4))
 (segment (start 166.156 122.301) (end 166.156 129.413) (width 0.76) (layer "B.Cu") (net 4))
 (segment (start 166.343 69.188) (end 165.581 69.188) (width 0.76) (layer "B.Cu") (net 1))
 (segment (start 162.439 69.188) (end 165.581 69.188) (width 0.76) (layer "B.Cu") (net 1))
 (segment (start 168.783 71.628) (end 166.343 69.188) (width 0.76) (layer "B.Cu") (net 1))
 (segment (start 166.751 79.502) (end 162.941 79.502) (width 0.76) (layer "B.Cu") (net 2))
 (segment (start 162.941 79.502) (end 159.893 76.454) (width 0.76) (layer "B.Cu") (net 2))
 (segment (start 168.783 81.534) (end 166.751 79.502) (width 0.76) (layer "B.Cu") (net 2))
 (segment (start 168.783 81.534) (end 168.783 86.868) (width 0.76) (layer "B.Cu") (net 2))
 (segment (start 168.656 115.196) (end 168.663 115.189) (width 0.76) (layer "B.Cu") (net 3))
 (segment (start 133.554 67.233) (end 135.594 67.233) (width 0.76) (layer "B.Cu") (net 3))
 (segment (start 146.431 121.666) (end 144.018 119.253) (width 0.76) (layer "B.Cu") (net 3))
 (segment (start 146.431 122.682) (end 146.431 121.666) (width 0.76) (layer "B.Cu") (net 3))
 (segment (start 131.191 115.062) (end 131.191 69.596) (width 0.76) (layer "B.Cu") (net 3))
 (segment (start 168.656 122.301) (end 168.656 115.196) (width 0.76) (layer "B.Cu") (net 3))
 (segment (start 163.83 134.239) (end 157.988 134.239) (width 0.76) (layer "B.Cu") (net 3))
 (segment (start 144.018 119.253) (end 135.382 119.253) (width 0.76) (layer "B.Cu") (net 3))
 (segment (start 131.191 115.062) (end 133.052 116.923) (width 0.76) (layer "B.Cu") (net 3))
 (segment (start 131.191 69.596) (end 133.554 67.233) (width 0.76) (layer "B.Cu") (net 3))
 (segment (start 168.656 129.413) (end 163.83 134.239) (width 0.76) (layer "B.Cu") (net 3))
 (segment (start 168.656 122.301) (end 168.656 129.413) (width 0.76) (layer "B.Cu") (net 3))
 (segment (start 157.988 134.239) (end 146.431 122.682) (width 0.76) (layer "B.Cu") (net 3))
 (segment (start 133.052 116.923) (end 135.382 119.253) (width 0.76) (layer "B.Cu") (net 3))
 (segment (start 151.257 93.056) (end 153.374 95.173) (width 0.76) (layer "B.Cu") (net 31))
 (segment (start 151.257 76.454) (end 151.257 93.056) (width 0.76) (layer "B.Cu") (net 31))
 (segment (start 162.433 83.82) (end 162.433 82.042) (width 0.76) (layer "B.Cu") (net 31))
 (segment (start 155.321 74.93) (end 152.781 74.93) (width 0.76) (layer "B.Cu") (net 31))
 (segment (start 152.781 74.93) (end 151.257 76.454) (width 0.76) (layer "B.Cu") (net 31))
 (segment (start 162.433 82.042) (end 155.321 74.93) (width 0.76) (layer "B.Cu") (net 31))
 (segment (start 159.893 87.884) (end 157.861 85.852) (width 0.76) (layer "B.Cu") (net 38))
 (segment (start 157.861 85.852) (end 157.861 81.88) (width 0.76) (layer "B.Cu") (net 38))
 (segment (start 157.861 81.88) (end 153.374 77.393) (width 0.76) (layer "B.Cu") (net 38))
 (segment (start 159.639 90.678) (end 159.639 91.44) (width 0.76) (layer "B.Cu") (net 38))
 (segment (start 169.545 91.186) (end 167.005 91.186) (width 0.76) (layer "B.Cu") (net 38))
 (segment (start 161.163 89.154) (end 159.639 90.678) (width 0.76) (layer "B.Cu") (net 38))
 (segment (start 164.973 89.154) (end 161.163 89.154) (width 0.76) (layer "B.Cu") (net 38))
 (segment (start 161.163 89.154) (end 159.893 87.884) (width 0.76) (layer "B.Cu") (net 38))
 (segment (start 167.005 91.186) (end 164.973 89.154) (width 0.76) (layer "B.Cu") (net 38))
 (segment (start 159.639 91.44) (end 159.639 98.806) (width 0.76) (layer "B.Cu") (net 38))
 (segment (start 160.478 72.313) (end 153.374 72.313) (width 0.76) (layer "B.Cu") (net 30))
 (segment (start 162.393 76.454) (end 162.393 74.228) (width 0.76) (layer "B.Cu") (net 30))
 (segment (start 153.184 97.713) (end 153.374 97.713) (width 0.76) (layer "B.Cu") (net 30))
 (segment (start 160.401 100.838) (end 157.861 100.838) (width 0.76) (layer "B.Cu") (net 30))
 (segment (start 154.736 97.713) (end 157.861 100.838) (width 0.76) (layer "B.Cu") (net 30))
 (segment (start 162.139 99.1) (end 160.401 100.838) (width 0.76) (layer "B.Cu") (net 30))
 (segment (start 153.451 97.79) (end 153.374 97.713) (width 0.76) (layer "B.Cu") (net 30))
 (segment (start 153.374 97.713) (end 154.736 97.713) (width 0.76) (layer "B.Cu") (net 30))
 (segment (start 162.139 98.806) (end 162.139 99.1) (width 0.25) (layer "B.Cu") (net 30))
 (segment (start 162.393 74.228) (end 160.478 72.313) (width 0.76) (layer "B.Cu") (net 30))
 (segment (start 153.377 97.71) (end 153.374 97.713) (width 0.76) (layer "B.Cu") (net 30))
 (segment (start 162.139 98.806) (end 162.139 91.44) (width 0.76) (layer "B.Cu") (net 30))
 (segment (start 164.639 98.806) (end 164.639 91.44) (width 0.76) (layer "B.Cu") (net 29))
 (segment (start 153.374 100.253) (end 155.229 102.108) (width 0.76) (layer "B.Cu") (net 29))
 (segment (start 164.639 98.806) (end 161.337 102.108) (width 0.76) (layer "B.Cu") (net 29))
 (segment (start 167.005 98.806) (end 169.545 101.346) (width 0.76) (layer "B.Cu") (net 29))
 (segment (start 164.639 98.886) (end 164.639 98.552) (width 0.76) (layer "B.Cu") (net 29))
 (segment (start 164.639 98.806) (end 167.005 98.806) (width 0.76) (layer "B.Cu") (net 29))
 (segment (start 161.337 102.108) (end 155.229 102.108) (width 0.76) (layer "B.Cu") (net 29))
 (segment (start 157.313 105.333) (end 160.672 108.692) (width 0.76) (layer "B.Cu") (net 27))
 (segment (start 153.374 105.333) (end 157.313 105.333) (width 0.76) (layer "B.Cu") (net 27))
 (segment (start 167.64 112.268) (end 164.084 112.268) (width 0.76) (layer "B.Cu") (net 40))
 (segment (start 161.163 115.189) (end 161.163 122.294) (width 0.76) (layer "B.Cu") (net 40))
 (segment (start 159.939 69.188) (end 162.579 66.548) (width 0.76) (layer "B.Cu") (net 40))
 (segment (start 171.831 87.122) (end 171.831 104.648) (width 0.76) (layer "B.Cu") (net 40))
 (segment (start 153.959 69.188) (end 153.374 69.773) (width 0.76) (layer "B.Cu") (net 40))
 (segment (start 162.579 66.548) (end 167.259 66.548) (width 0.76) (layer "B.Cu") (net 40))
 (segment (start 164.973 86.146) (end 162.259 86.146) (width 0.76) (layer "B.Cu") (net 40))
 (segment (start 171.831 104.648) (end 171.831 108.077) (width 0.76) (layer "B.Cu") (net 40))
 (segment (start 161.163 122.294) (end 161.156 122.301) (width 0.76) (layer "B.Cu") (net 40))
 (segment (start 167.727 88.9) (end 170.053 88.9) (width 0.76) (layer "B.Cu") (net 40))
 (segment (start 164.084 112.268) (end 161.163 115.189) (width 0.76) (layer "B.Cu") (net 40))
 (segment (start 171.831 104.648) (end 169.582 104.648) (width 0.76) (layer "B.Cu") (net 40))
 (segment (start 161.156 122.301) (end 161.156 129.413) (width 0.76) (layer "B.Cu") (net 40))
 (segment (start 169.582 104.648) (end 168.038 106.192) (width 0.76) (layer "B.Cu") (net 40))
 (segment (start 171.831 71.12) (end 171.831 87.122) (width 0.76) (layer "B.Cu") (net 40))
 (segment (start 164.973 86.146) (end 167.727 88.9) (width 0.76) (layer "B.Cu") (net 40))
 (segment (start 159.801 83.82) (end 159.933 83.82) (width 0.25) (layer "B.Cu") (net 40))
 (segment (start 167.259 66.548) (end 171.831 71.12) (width 0.76) (layer "B.Cu") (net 40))
 (segment (start 154.686 122.301) (end 154.051 121.666) (width 0.76) (layer "B.Cu") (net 40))
 (segment (start 171.831 108.077) (end 167.64 112.268) (width 0.76) (layer "B.Cu") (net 40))
 (segment (start 161.156 122.301) (end 154.686 122.301) (width 0.76) (layer "B.Cu") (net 40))
 (segment (start 168.038 106.192) (end 160.672 106.192) (width 0.76) (layer "B.Cu") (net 40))
 (segment (start 159.939 69.188) (end 153.959 69.188) (width 0.76) (layer "B.Cu") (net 40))
 (segment (start 170.053 88.9) (end 171.831 87.122) (width 0.76) (layer "B.Cu") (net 40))
 (segment (start 162.259 86.146) (end 159.933 83.82) (width 0.76) (layer "B.Cu") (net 40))
 (segment (start 163.656 129.413) (end 163.656 130.095) (width 0.76) (layer "B.Cu") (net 25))
 (segment (start 163.656 122.301) (end 163.656 115.196) (width 0.76) (layer "B.Cu") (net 25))
 (segment (start 155.702 117.475) (end 151.511 121.666) (width 0.76) (layer "B.Cu") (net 25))
 (segment (start 162.179 131.572) (end 159.893 131.572) (width 0.76) (layer "B.Cu") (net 25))
 (segment (start 155.702 112.741) (end 155.702 117.475) (width 0.76) (layer "B.Cu") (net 25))
 (segment (start 163.663 115.189) (end 163.663 114.768) (width 0.25) (layer "B.Cu") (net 25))
 (segment (start 159.893 131.572) (end 151.511 123.19) (width 0.76) (layer "B.Cu") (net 25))
 (segment (start 163.656 130.095) (end 162.179 131.572) (width 0.76) (layer "B.Cu") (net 25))
 (segment (start 151.511 123.19) (end 151.511 121.666) (width 0.76) (layer "B.Cu") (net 25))
 (segment (start 152.974 110.413) (end 153.374 110.413) (width 0.76) (layer "B.Cu") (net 25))
 (segment (start 163.656 115.196) (end 163.663 115.189) (width 0.76) (layer "B.Cu") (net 25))
 (segment (start 163.656 122.301) (end 163.656 129.413) (width 0.76) (layer "B.Cu") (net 25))
 (segment (start 153.374 110.413) (end 153.466 110.413) (width 0.76) (layer "B.Cu") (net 25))
 (segment (start 153.374 110.413) (end 155.702 112.741) (width 0.76) (layer "B.Cu") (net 25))
 (segment (start 155.244 107.873) (end 158.115 110.744) (width 0.76) (layer "B.Cu") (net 26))
 (segment (start 153.374 107.873) (end 155.244 107.873) (width 0.76) (layer "B.Cu") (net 26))
 (segment (start 158.115 110.744) (end 165.986 110.744) (width 0.76) (layer "B.Cu") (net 26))
 (segment (start 165.986 110.744) (end 168.038 108.692) (width 0.76) (layer "B.Cu") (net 26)))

